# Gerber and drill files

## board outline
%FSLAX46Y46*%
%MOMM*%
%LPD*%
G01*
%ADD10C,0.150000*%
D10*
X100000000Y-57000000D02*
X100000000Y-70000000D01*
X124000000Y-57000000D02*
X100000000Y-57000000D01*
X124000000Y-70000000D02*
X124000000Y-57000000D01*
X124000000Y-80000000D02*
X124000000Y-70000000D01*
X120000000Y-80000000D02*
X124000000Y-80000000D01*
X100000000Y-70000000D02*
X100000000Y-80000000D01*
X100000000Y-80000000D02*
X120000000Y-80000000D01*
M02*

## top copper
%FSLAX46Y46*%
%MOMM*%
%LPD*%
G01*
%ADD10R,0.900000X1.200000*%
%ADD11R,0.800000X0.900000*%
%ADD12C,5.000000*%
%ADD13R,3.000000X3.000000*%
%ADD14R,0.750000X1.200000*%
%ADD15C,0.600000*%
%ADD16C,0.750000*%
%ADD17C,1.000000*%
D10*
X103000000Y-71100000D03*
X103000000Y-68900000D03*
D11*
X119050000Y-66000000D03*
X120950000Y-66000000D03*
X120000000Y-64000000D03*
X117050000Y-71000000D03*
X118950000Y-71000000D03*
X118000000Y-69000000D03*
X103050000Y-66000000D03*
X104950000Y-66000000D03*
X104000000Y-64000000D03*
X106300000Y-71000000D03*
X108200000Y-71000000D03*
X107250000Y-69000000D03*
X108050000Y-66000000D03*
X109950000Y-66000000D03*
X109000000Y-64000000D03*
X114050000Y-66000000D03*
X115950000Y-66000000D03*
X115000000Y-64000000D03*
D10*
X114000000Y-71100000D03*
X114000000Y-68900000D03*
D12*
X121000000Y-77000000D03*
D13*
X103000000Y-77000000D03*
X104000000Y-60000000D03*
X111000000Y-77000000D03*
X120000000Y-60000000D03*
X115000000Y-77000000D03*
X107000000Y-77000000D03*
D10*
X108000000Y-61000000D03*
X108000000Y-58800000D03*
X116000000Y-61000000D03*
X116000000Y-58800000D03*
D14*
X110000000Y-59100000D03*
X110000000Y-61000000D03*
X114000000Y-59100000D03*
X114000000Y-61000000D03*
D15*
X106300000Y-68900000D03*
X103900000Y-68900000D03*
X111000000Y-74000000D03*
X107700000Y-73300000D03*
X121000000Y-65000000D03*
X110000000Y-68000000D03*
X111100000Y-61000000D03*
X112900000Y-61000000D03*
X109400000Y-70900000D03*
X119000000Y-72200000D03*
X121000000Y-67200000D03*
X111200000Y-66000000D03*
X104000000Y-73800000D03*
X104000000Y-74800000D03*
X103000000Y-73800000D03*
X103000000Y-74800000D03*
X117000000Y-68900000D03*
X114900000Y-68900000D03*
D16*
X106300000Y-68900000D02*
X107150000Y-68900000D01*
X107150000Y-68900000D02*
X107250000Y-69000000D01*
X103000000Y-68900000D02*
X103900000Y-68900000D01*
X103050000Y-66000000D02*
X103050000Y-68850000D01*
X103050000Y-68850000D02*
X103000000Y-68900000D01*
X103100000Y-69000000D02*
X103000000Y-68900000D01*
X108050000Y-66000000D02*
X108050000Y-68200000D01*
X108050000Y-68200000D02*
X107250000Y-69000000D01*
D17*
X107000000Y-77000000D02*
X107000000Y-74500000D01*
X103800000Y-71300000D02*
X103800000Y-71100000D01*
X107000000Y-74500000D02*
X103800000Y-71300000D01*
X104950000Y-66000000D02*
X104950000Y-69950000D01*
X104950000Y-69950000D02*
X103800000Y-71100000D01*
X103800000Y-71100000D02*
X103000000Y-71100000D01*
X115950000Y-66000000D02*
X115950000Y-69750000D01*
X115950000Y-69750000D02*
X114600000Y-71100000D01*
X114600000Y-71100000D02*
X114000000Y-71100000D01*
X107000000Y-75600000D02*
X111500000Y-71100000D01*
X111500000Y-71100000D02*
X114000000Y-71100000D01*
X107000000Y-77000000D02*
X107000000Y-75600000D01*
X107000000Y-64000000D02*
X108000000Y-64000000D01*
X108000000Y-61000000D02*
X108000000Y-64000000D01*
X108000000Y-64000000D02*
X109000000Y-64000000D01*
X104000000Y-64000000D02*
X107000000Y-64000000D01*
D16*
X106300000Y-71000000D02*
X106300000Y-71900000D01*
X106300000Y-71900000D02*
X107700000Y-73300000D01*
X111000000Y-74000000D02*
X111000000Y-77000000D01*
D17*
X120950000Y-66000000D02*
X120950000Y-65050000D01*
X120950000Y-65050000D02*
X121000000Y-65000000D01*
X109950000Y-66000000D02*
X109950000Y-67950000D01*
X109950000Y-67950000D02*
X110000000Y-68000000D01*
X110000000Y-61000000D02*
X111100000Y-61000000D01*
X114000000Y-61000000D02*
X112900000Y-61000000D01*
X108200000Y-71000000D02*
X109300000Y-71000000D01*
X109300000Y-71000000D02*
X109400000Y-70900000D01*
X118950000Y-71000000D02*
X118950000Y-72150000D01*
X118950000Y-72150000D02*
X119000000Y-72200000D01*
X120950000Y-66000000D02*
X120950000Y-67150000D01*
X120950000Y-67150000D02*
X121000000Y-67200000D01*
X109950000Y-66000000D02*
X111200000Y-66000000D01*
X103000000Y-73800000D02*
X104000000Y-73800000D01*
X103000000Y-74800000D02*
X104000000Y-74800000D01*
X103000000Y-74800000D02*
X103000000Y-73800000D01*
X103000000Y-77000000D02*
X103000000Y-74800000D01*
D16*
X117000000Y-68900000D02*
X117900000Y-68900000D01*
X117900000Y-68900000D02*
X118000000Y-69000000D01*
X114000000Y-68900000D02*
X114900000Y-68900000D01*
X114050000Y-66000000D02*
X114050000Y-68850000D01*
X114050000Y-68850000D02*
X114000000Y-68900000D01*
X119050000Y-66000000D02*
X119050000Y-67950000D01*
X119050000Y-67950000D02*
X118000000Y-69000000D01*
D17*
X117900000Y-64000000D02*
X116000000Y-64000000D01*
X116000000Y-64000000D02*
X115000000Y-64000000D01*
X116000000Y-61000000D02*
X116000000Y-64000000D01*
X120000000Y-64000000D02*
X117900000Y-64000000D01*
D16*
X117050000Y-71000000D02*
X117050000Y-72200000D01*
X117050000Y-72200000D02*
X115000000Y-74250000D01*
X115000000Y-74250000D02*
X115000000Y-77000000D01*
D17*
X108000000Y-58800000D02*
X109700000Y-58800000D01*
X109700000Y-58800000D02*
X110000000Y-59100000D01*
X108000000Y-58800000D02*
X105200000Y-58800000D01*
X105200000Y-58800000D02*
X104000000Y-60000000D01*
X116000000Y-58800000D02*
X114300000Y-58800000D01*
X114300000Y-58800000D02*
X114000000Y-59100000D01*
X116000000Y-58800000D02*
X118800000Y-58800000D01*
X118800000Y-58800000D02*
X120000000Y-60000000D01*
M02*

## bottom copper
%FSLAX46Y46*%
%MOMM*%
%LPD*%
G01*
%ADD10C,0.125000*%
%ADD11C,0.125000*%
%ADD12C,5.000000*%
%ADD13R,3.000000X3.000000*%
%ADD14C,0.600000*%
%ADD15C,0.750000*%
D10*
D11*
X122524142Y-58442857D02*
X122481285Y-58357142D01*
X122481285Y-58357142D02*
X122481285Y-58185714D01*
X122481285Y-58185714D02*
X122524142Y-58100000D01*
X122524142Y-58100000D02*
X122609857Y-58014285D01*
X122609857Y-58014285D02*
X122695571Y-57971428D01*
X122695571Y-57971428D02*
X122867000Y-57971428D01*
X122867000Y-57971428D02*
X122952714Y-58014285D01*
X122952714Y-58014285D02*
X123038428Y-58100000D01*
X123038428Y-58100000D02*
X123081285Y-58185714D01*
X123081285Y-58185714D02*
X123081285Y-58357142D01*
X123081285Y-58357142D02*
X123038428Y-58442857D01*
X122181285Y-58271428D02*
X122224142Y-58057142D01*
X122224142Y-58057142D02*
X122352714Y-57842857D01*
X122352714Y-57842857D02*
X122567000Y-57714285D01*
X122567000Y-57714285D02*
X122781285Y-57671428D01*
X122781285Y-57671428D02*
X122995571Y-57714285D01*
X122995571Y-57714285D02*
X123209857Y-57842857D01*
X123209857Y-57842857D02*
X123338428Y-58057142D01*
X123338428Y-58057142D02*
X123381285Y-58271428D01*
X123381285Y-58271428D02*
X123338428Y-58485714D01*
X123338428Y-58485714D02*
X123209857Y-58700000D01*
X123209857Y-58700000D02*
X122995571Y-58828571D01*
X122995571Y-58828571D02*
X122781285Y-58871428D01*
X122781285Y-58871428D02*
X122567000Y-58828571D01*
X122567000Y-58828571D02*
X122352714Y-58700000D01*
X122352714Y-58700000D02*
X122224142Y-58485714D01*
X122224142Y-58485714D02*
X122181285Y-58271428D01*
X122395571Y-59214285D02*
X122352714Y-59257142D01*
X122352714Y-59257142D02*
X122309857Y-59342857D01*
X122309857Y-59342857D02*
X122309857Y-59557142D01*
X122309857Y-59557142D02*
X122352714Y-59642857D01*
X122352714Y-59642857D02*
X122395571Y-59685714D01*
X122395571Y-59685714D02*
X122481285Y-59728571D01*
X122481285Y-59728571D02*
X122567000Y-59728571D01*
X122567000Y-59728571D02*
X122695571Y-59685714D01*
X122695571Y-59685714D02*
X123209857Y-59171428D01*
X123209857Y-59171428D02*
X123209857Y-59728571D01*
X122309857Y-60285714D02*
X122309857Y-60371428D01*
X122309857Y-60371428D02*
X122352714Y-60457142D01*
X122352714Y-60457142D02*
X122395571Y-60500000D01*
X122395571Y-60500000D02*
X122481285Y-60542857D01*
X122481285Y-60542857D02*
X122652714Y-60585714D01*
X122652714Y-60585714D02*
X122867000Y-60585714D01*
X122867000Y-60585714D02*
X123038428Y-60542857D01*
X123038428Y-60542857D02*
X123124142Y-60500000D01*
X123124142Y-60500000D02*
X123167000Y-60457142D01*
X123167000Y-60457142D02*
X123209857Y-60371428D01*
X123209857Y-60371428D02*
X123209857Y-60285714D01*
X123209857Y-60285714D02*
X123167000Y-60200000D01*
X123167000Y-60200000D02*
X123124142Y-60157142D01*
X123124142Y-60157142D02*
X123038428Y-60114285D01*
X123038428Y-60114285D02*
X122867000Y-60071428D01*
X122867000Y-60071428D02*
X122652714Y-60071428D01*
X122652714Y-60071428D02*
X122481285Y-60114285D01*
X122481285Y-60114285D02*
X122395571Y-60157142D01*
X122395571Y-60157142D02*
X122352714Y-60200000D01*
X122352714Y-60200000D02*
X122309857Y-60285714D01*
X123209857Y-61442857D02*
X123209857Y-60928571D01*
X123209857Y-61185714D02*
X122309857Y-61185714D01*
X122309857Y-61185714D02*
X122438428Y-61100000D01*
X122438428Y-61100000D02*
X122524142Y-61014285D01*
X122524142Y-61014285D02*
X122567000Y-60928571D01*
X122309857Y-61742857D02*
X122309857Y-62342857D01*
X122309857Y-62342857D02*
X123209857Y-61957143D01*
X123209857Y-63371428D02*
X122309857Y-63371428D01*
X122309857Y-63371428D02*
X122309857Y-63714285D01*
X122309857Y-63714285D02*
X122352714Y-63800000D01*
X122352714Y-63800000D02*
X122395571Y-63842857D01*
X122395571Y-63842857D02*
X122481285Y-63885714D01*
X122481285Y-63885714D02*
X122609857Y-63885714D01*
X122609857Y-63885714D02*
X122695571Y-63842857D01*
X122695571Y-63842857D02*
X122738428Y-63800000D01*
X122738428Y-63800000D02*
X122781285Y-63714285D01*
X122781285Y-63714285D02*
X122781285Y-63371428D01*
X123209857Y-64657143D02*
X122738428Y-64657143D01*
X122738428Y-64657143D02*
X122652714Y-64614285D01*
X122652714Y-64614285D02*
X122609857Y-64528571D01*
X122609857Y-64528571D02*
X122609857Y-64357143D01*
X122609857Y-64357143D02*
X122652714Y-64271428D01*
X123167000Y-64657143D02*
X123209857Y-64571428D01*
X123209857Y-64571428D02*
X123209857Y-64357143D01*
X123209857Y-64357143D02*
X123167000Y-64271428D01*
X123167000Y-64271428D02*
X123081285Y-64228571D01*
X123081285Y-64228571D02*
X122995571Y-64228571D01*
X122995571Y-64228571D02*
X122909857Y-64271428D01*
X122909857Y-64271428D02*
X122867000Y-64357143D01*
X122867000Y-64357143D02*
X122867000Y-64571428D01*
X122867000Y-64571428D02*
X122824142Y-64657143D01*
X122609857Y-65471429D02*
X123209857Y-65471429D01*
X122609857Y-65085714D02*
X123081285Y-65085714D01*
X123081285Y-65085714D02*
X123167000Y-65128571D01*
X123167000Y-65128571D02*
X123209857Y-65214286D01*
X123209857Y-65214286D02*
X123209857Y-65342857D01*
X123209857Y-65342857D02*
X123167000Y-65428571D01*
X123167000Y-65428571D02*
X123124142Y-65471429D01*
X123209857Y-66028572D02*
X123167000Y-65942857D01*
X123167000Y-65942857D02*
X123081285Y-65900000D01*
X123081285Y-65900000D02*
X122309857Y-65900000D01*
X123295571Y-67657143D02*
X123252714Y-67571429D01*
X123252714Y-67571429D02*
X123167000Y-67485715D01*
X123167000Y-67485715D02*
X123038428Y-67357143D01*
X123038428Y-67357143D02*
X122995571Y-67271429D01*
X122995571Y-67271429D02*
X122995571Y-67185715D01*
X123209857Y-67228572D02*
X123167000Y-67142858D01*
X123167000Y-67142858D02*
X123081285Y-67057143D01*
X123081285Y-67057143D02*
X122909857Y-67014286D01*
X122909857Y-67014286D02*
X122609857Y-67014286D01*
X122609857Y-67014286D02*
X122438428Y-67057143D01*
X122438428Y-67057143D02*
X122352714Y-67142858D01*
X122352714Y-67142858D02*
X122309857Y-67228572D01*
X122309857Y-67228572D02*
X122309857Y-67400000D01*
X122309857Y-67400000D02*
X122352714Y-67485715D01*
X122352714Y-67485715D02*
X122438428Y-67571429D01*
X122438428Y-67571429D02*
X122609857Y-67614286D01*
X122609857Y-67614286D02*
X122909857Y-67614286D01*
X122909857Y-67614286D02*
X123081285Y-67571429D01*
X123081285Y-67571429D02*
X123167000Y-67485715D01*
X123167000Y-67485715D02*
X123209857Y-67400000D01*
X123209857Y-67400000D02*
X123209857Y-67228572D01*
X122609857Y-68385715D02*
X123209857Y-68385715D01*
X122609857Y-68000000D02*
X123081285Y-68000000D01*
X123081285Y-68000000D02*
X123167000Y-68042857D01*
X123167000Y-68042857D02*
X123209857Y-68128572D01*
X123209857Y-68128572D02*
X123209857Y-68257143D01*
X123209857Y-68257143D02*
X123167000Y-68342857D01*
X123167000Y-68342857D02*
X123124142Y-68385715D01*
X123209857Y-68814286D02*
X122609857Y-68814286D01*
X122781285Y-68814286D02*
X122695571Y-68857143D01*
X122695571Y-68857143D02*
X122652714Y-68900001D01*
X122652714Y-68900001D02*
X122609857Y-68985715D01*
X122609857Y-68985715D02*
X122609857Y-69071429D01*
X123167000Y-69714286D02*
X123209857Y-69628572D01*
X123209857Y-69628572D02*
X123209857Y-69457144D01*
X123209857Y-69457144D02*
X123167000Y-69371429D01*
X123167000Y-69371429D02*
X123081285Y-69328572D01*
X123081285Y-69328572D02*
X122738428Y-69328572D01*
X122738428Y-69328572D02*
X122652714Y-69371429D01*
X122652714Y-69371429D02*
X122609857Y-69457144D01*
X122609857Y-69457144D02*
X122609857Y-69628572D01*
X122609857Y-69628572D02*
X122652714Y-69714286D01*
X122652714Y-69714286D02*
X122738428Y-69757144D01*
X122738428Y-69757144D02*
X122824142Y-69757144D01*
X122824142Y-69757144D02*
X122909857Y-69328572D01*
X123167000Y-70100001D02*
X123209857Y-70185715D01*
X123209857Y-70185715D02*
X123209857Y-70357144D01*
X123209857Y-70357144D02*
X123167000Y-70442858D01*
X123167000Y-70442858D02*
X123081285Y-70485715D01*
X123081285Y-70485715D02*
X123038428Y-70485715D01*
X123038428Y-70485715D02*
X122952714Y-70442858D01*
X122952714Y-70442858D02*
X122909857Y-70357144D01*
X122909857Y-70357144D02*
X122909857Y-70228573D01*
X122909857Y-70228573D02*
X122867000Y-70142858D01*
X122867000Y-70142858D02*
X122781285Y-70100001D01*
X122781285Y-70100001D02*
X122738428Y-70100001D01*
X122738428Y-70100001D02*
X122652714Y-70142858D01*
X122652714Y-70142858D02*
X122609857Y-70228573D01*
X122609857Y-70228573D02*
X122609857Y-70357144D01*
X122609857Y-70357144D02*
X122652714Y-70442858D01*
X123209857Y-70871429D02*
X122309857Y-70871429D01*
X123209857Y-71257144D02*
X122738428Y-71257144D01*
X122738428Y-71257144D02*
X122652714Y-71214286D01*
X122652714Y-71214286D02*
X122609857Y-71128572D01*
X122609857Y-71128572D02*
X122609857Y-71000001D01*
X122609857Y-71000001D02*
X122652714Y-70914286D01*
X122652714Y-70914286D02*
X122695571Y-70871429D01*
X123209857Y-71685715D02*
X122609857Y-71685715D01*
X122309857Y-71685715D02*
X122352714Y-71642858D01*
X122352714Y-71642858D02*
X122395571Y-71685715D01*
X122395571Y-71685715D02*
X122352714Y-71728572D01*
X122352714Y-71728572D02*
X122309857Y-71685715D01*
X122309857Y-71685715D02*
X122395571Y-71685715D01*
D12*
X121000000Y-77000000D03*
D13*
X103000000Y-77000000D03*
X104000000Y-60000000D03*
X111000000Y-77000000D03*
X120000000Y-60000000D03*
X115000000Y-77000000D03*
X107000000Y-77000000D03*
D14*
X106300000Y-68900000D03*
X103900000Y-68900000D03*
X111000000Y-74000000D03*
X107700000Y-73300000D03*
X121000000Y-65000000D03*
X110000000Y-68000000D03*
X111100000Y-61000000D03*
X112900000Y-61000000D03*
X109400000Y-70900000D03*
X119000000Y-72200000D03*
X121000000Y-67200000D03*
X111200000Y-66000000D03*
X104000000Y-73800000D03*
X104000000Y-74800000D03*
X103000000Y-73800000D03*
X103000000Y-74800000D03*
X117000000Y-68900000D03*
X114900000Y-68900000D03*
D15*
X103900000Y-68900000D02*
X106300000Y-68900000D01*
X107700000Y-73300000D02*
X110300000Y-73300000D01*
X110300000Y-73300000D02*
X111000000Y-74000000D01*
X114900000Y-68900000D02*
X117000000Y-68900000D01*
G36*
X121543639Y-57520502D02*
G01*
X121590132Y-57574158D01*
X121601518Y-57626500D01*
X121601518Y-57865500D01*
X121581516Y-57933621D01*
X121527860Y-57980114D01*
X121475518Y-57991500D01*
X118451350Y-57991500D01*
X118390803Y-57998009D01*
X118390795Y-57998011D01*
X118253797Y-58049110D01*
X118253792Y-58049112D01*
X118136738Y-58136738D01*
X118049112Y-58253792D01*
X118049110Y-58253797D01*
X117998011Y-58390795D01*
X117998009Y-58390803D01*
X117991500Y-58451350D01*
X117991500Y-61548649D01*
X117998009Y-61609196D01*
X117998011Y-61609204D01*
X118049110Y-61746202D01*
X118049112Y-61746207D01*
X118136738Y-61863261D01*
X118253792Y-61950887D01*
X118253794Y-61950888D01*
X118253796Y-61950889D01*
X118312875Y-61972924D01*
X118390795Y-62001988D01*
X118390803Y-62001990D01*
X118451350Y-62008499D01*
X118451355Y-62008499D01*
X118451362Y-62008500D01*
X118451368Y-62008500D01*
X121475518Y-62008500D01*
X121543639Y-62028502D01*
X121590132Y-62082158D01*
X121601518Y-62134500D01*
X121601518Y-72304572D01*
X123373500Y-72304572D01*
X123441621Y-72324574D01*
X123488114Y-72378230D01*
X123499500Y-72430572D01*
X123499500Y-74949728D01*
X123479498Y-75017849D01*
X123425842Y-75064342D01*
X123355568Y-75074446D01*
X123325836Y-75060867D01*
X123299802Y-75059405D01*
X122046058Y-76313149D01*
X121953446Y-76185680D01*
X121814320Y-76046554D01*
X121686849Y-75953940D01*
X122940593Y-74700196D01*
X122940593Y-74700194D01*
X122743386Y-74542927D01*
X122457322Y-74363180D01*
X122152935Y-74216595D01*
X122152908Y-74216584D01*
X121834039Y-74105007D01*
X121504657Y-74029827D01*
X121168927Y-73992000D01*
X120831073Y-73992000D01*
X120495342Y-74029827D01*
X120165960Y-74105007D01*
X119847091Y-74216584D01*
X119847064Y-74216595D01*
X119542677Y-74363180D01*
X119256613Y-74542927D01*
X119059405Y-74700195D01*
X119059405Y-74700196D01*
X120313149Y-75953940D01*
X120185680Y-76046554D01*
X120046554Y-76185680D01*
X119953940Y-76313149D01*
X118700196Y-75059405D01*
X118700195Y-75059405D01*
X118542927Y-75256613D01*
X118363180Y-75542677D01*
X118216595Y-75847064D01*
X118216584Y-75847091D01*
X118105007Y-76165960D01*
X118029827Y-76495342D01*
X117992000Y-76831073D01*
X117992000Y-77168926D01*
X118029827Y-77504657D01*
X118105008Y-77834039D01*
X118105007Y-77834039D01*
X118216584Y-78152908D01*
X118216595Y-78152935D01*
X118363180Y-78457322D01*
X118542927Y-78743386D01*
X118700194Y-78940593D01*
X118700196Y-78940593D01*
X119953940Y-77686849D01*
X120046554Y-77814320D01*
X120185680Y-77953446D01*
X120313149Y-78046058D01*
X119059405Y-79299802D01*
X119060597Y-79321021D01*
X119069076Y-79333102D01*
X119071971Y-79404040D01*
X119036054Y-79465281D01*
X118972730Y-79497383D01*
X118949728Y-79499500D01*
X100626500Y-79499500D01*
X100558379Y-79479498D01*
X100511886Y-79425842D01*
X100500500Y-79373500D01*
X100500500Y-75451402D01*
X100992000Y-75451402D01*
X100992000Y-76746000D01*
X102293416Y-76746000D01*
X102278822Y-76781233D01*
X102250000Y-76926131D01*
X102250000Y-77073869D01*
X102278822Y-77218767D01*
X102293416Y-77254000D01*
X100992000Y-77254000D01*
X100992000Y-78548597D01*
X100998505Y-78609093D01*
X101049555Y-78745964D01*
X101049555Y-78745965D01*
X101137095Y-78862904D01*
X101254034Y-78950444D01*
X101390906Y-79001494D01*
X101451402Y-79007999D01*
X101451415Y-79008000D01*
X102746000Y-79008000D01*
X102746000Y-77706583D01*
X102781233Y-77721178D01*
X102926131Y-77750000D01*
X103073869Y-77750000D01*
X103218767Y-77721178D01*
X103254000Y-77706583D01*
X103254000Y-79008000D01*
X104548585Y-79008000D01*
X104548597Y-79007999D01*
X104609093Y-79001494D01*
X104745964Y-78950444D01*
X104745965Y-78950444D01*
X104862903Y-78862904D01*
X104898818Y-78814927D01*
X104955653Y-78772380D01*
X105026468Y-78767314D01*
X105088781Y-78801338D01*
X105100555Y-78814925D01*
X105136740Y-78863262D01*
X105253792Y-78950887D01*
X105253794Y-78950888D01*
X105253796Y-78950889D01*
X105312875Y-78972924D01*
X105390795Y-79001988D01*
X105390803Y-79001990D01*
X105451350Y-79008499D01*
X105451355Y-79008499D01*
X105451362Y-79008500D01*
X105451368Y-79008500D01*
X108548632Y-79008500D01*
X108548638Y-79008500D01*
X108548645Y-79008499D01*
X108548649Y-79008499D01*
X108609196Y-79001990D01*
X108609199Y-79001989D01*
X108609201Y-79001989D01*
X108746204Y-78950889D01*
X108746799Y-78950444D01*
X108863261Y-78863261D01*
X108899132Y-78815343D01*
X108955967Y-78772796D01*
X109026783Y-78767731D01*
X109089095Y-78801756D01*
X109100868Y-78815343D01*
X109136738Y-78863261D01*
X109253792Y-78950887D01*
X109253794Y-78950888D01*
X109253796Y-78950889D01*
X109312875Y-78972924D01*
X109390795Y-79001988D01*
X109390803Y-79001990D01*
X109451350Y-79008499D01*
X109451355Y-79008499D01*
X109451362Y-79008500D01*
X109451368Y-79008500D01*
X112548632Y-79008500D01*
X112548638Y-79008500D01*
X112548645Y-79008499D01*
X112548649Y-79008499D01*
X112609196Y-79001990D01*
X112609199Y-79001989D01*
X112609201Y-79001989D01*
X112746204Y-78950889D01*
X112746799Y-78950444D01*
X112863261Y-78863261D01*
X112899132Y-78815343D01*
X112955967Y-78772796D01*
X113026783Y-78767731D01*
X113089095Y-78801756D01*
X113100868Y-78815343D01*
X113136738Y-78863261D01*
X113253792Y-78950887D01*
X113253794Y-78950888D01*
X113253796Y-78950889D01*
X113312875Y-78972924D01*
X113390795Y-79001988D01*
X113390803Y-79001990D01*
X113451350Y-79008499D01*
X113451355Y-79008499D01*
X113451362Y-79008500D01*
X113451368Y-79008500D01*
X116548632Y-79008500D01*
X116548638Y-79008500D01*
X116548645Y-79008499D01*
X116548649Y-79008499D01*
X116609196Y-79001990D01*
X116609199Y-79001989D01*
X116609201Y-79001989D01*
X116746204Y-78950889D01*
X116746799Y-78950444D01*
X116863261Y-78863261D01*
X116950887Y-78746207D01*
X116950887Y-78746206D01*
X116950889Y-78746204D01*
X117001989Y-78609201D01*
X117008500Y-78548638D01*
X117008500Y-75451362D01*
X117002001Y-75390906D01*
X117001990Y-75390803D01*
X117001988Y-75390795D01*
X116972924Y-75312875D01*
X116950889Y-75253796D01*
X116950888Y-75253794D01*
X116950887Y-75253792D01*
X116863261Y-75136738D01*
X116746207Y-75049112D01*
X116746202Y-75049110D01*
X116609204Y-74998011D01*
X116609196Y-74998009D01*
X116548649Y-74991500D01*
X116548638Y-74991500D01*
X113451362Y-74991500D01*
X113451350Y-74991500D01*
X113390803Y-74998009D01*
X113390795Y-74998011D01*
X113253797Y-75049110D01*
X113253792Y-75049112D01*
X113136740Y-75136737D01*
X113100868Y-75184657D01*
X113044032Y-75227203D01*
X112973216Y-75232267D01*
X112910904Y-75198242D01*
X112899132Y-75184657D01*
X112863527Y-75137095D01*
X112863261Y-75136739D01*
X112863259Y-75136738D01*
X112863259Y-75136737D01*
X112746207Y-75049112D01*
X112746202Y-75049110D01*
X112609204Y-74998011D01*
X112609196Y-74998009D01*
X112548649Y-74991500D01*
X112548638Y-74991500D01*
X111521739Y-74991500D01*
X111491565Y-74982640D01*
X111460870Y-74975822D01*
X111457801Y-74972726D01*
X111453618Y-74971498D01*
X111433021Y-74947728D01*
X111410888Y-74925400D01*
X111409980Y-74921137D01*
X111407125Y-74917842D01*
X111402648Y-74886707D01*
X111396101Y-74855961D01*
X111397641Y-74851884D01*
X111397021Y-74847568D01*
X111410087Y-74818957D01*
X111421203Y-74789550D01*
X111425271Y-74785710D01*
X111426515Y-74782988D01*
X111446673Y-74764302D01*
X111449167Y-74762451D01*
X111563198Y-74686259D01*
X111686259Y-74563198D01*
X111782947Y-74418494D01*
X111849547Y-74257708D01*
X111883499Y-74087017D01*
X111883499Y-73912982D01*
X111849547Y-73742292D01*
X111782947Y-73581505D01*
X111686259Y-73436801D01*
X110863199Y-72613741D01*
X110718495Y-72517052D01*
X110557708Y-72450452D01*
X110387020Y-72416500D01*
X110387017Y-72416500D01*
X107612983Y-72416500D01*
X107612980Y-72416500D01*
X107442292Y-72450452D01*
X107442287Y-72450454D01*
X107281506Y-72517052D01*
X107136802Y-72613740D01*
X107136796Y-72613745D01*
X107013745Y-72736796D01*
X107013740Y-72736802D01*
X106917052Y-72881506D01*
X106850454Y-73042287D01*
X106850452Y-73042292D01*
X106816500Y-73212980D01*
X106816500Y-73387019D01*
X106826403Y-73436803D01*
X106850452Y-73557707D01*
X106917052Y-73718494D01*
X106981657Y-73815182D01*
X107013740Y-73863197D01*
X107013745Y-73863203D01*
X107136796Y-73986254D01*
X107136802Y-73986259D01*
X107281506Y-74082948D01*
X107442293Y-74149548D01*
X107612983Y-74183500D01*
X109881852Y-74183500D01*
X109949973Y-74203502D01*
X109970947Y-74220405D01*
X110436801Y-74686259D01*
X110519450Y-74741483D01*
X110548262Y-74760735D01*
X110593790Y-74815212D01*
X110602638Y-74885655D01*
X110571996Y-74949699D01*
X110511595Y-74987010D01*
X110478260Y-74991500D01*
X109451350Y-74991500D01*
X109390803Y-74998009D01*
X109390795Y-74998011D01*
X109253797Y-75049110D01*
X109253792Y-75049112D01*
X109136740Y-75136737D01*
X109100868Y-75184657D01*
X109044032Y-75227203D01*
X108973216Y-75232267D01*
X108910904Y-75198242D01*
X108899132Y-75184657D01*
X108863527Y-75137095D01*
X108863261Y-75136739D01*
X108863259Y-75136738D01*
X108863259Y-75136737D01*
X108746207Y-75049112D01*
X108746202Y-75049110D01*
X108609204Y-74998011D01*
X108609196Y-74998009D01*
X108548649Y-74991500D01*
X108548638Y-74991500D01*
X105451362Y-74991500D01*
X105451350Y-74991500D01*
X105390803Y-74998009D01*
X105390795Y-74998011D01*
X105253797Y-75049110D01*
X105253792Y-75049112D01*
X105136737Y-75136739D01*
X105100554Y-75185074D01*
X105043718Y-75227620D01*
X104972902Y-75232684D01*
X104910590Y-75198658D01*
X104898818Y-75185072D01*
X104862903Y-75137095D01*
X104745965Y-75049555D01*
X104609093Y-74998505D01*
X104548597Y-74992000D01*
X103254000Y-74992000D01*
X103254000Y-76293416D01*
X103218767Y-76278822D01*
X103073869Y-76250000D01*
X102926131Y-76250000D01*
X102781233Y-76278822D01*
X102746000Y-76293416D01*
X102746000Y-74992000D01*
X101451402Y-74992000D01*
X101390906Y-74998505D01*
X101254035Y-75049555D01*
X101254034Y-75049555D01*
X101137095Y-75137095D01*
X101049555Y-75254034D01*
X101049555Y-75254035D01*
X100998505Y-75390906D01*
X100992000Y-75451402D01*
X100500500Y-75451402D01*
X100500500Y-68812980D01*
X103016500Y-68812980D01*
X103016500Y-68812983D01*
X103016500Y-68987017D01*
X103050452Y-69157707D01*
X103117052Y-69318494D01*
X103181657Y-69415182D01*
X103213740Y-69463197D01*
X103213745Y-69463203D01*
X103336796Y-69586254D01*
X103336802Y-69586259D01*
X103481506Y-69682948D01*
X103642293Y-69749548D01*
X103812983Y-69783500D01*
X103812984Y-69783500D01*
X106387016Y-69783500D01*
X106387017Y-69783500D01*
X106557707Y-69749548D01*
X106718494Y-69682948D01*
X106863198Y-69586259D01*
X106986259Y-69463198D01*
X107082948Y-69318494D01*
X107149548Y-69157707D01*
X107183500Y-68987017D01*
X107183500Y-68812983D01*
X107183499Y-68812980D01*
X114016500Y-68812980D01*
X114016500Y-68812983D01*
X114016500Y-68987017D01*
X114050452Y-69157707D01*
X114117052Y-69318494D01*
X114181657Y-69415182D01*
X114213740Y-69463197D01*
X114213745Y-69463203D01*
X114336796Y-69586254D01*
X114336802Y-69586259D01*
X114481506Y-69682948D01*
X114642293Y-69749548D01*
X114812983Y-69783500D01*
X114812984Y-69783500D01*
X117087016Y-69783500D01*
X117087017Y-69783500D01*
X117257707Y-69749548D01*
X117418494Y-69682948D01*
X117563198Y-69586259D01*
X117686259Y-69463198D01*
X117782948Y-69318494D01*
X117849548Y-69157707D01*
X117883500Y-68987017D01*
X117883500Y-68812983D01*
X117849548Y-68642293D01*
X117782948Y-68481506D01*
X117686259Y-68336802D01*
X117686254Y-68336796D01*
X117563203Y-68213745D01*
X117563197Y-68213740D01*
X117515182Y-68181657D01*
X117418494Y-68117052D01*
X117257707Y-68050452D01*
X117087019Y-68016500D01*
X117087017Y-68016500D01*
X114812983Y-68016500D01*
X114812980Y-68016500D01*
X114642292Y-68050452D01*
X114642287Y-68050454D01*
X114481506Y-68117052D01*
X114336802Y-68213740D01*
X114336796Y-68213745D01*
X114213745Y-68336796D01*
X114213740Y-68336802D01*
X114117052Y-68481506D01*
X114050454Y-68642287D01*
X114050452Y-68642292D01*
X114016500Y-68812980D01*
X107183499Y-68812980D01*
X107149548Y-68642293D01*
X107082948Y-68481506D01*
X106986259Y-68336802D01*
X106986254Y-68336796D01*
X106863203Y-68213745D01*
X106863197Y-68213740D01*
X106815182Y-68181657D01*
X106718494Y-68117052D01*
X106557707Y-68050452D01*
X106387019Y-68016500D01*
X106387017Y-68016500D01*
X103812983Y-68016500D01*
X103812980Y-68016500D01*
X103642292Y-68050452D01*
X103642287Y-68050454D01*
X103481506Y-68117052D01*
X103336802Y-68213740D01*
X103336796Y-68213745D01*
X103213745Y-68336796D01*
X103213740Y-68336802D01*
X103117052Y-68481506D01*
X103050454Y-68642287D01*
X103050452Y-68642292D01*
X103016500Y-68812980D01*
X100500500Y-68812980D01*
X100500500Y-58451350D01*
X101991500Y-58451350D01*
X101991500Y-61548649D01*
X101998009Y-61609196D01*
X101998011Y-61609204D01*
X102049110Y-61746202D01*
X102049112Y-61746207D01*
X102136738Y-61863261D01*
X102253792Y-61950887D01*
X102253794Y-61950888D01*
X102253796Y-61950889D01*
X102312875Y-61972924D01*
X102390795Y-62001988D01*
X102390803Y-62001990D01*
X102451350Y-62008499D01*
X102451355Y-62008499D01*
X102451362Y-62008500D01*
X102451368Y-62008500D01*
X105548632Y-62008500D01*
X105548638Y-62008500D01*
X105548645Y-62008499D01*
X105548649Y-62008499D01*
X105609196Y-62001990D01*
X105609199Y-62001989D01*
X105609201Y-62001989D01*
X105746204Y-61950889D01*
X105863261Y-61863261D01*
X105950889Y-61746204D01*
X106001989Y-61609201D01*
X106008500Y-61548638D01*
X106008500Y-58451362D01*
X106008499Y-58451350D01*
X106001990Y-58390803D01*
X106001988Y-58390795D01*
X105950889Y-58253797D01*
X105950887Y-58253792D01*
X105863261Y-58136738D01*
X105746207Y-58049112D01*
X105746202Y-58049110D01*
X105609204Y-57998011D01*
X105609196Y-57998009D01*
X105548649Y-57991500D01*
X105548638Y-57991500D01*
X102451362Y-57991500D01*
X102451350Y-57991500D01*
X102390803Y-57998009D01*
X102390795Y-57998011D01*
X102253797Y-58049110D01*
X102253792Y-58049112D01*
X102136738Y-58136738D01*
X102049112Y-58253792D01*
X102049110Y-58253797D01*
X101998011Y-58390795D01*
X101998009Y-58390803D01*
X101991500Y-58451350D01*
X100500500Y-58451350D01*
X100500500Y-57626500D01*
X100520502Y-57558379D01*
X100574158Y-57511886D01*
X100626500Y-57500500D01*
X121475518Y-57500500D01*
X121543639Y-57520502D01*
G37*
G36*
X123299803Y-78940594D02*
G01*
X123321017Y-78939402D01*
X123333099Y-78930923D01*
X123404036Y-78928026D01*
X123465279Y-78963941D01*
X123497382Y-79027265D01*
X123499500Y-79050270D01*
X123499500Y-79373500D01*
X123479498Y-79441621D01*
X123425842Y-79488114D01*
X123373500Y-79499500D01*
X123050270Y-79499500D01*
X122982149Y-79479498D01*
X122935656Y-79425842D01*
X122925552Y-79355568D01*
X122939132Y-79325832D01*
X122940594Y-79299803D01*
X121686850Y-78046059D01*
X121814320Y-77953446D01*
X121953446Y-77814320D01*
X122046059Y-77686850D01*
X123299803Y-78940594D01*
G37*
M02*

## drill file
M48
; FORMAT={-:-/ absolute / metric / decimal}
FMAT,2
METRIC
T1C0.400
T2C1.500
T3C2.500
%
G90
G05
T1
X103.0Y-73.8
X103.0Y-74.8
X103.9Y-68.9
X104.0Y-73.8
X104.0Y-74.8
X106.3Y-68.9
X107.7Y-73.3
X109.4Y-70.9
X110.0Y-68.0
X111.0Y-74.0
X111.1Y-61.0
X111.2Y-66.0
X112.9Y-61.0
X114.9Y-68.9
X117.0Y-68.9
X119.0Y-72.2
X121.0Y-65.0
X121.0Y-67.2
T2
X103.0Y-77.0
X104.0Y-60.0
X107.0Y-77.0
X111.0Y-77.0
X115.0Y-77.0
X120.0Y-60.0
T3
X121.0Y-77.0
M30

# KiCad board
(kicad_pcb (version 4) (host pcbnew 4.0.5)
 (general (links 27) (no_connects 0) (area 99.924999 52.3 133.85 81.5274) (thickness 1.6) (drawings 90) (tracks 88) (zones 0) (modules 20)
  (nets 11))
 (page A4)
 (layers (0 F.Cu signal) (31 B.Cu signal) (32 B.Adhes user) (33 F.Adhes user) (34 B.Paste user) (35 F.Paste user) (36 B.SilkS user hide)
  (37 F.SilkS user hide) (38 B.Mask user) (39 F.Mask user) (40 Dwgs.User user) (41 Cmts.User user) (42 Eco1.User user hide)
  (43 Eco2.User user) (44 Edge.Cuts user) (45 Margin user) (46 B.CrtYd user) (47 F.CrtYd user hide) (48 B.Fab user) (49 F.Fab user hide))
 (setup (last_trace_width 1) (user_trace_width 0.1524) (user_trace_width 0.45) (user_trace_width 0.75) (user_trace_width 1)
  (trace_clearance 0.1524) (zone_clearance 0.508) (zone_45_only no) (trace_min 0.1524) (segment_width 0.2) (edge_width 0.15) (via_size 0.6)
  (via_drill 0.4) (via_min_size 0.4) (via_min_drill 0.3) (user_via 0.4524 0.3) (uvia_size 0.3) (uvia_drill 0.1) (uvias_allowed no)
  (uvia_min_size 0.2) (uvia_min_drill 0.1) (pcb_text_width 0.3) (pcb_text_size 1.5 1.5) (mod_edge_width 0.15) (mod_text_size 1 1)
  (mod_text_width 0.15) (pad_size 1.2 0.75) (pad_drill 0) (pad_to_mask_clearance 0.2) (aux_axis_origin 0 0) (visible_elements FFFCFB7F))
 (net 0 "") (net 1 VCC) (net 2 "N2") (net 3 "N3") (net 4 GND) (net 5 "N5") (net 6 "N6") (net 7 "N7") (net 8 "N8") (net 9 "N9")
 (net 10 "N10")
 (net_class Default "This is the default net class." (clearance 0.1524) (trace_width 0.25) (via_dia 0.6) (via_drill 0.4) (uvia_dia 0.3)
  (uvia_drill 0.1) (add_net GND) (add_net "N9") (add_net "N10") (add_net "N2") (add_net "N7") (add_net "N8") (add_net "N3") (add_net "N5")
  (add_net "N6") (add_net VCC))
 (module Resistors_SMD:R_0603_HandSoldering (layer F.Cu) (at 103 70 90)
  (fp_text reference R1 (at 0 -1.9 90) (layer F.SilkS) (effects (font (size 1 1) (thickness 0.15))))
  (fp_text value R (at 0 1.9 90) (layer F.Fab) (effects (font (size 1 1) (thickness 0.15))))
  (pad 1 smd rect (at -1.1 0 90) (size 1.2 0.9) (layers F.Cu F.Paste F.Mask) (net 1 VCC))
  (pad 2 smd rect (at 1.1 0 90) (size 1.2 0.9) (layers F.Cu F.Paste F.Mask) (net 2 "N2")))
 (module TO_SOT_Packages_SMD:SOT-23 (layer F.Cu) (at 120 65 90)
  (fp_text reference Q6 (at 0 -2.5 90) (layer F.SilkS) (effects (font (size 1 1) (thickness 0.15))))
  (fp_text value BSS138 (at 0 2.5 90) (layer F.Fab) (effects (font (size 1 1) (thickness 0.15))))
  (pad 1 smd rect (at -1 -0.95 90) (size 0.9 0.8) (layers F.Cu F.Paste F.Mask) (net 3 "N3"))
  (pad 2 smd rect (at -1 0.95 90) (size 0.9 0.8) (layers F.Cu F.Paste F.Mask) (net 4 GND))
  (pad 3 smd rect (at 1 0 90) (size 0.9 0.8) (layers F.Cu F.Paste F.Mask) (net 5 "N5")))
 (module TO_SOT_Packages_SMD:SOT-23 (layer F.Cu) (at 118 70 90)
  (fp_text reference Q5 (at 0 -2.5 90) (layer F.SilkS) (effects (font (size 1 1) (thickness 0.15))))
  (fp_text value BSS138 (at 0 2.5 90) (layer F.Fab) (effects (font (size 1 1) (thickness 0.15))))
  (pad 1 smd rect (at -1 -0.95 90) (size 0.9 0.8) (layers F.Cu F.Paste F.Mask) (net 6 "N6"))
  (pad 2 smd rect (at -1 0.95 90) (size 0.9 0.8) (layers F.Cu F.Paste F.Mask) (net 4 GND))
  (pad 3 smd rect (at 1 0 90) (size 0.9 0.8) (layers F.Cu F.Paste F.Mask) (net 3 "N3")))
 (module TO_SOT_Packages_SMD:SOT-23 (layer F.Cu) (at 104 65 90)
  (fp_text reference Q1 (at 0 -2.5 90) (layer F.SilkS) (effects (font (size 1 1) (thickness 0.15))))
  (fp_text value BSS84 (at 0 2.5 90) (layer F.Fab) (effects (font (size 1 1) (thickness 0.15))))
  (pad 1 smd rect (at -1 -0.95 90) (size 0.9 0.8) (layers F.Cu F.Paste F.Mask) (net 2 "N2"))
  (pad 2 smd rect (at -1 0.95 90) (size 0.9 0.8) (layers F.Cu F.Paste F.Mask) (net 1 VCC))
  (pad 3 smd rect (at 1 0 90) (size 0.9 0.8) (layers F.Cu F.Paste F.Mask) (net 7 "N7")))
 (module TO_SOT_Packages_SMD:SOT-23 (layer F.Cu) (at 107.25 70 90)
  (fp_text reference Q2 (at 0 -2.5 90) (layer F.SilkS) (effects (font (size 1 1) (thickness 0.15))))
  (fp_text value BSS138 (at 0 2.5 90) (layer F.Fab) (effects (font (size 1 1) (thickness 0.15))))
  (pad 1 smd rect (at -1 -0.95 90) (size 0.9 0.8) (layers F.Cu F.Paste F.Mask) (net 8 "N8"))
  (pad 2 smd rect (at -1 0.95 90) (size 0.9 0.8) (layers F.Cu F.Paste F.Mask) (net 4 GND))
  (pad 3 smd rect (at 1 0 90) (size 0.9 0.8) (layers F.Cu F.Paste F.Mask) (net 2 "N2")))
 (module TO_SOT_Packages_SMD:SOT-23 (layer F.Cu) (at 109 65 90)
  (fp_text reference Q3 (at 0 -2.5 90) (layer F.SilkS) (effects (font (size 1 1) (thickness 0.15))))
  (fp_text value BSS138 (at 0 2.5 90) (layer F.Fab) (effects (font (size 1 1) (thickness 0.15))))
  (pad 1 smd rect (at -1 -0.95 90) (size 0.9 0.8) (layers F.Cu F.Paste F.Mask) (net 2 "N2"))
  (pad 2 smd rect (at -1 0.95 90) (size 0.9 0.8) (layers F.Cu F.Paste F.Mask) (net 4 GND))
  (pad 3 smd rect (at 1 0 90) (size 0.9 0.8) (layers F.Cu F.Paste F.Mask) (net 7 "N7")))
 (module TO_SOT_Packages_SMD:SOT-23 (layer F.Cu) (at 115 65 90)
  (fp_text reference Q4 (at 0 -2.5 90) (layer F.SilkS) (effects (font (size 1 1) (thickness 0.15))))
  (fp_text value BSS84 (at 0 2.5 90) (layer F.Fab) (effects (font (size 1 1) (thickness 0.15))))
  (pad 1 smd rect (at -1 -0.95 90) (size 0.9 0.8) (layers F.Cu F.Paste F.Mask) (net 3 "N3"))
  (pad 2 smd rect (at -1 0.95 90) (size 0.9 0.8) (layers F.Cu F.Paste F.Mask) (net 1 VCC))
  (pad 3 smd rect (at 1 0 90) (size 0.9 0.8) (layers F.Cu F.Paste F.Mask) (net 5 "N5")))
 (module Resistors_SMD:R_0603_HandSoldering (layer F.Cu) (at 114 70 90)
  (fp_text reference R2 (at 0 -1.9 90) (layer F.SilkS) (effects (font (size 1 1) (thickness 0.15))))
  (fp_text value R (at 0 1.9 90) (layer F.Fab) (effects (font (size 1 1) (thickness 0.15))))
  (pad 1 smd rect (at -1.1 0 90) (size 1.2 0.9) (layers F.Cu F.Paste F.Mask) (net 1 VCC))
  (pad 2 smd rect (at 1.1 0 90) (size 1.2 0.9) (layers F.Cu F.Paste F.Mask) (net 3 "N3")))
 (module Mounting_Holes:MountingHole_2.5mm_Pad (layer F.Cu) (at 121 77)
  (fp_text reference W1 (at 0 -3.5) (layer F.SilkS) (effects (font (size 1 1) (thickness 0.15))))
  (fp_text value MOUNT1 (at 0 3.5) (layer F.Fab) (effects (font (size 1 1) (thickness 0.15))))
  (pad 1 thru_hole circle (at 0 0) (size 5 5) (drill 2.5) (layers *.Cu *.Mask) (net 4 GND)))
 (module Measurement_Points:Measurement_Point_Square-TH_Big (layer F.Cu) (at 103 77)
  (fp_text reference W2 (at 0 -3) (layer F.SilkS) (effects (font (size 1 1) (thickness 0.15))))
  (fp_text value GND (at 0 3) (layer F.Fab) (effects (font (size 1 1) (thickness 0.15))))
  (pad 1 thru_hole rect (at 0 0) (size 3 3) (drill 1.5) (layers *.Cu *.Mask) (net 4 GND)))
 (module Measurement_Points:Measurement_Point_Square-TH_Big (layer F.Cu) (at 104 60)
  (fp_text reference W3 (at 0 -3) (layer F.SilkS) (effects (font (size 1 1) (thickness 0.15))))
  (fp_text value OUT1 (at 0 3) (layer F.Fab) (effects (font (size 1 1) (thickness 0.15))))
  (pad 1 thru_hole rect (at 0 0) (size 3 3) (drill 1.5) (layers *.Cu *.Mask) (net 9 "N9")))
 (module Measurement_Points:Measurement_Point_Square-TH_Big (layer F.Cu) (at 111 77)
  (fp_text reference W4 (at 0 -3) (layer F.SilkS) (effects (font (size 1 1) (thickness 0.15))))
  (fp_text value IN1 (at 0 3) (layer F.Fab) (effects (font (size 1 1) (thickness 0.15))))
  (pad 1 thru_hole rect (at 0 0) (size 3 3) (drill 1.5) (layers *.Cu *.Mask) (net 8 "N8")))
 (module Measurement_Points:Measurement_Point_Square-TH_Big (layer F.Cu) (at 120 60)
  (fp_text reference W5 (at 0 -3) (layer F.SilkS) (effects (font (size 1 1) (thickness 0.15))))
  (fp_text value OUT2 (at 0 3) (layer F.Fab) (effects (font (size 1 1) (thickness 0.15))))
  (pad 1 thru_hole rect (at 0 0) (size 3 3) (drill 1.5) (layers *.Cu *.Mask) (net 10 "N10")))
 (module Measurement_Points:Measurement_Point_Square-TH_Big (layer F.Cu) (at 115 77)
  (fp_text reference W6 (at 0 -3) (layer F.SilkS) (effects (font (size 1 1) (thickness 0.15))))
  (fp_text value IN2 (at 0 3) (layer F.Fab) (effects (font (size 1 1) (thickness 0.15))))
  (pad 1 thru_hole rect (at 0 0) (size 3 3) (drill 1.5) (layers *.Cu *.Mask) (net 6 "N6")))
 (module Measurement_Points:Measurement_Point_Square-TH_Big (layer F.Cu) (at 107 77)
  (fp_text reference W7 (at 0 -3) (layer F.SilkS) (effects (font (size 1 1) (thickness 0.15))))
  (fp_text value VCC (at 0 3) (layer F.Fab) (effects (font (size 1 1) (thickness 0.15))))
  (pad 1 thru_hole rect (at 0 0) (size 3 3) (drill 1.5) (layers *.Cu *.Mask) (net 1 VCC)))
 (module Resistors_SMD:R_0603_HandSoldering (layer F.Cu) (at 108 59.9 90)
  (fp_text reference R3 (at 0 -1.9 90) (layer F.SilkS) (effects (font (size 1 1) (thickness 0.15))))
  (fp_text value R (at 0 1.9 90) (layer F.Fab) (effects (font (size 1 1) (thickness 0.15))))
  (pad 1 smd rect (at -1.1 0 90) (size 1.2 0.9) (layers F.Cu F.Paste F.Mask) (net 7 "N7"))
  (pad 2 smd rect (at 1.1 0 90) (size 1.2 0.9) (layers F.Cu F.Paste F.Mask) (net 9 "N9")))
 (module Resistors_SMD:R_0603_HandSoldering (layer F.Cu) (at 116 59.9 90)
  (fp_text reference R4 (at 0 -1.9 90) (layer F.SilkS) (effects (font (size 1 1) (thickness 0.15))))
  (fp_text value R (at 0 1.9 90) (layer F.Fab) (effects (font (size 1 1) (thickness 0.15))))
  (pad 1 smd rect (at -1.1 0 90) (size 1.2 0.9) (layers F.Cu F.Paste F.Mask) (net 5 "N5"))
  (pad 2 smd rect (at 1.1 0 90) (size 1.2 0.9) (layers F.Cu F.Paste F.Mask) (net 10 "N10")))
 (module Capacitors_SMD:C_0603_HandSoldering (layer F.Cu) (at 110 60.05 270)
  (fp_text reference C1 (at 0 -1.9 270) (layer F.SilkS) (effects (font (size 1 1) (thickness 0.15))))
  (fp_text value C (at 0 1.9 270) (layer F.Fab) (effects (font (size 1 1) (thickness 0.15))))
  (pad 1 smd rect (at -0.95 0 270) (size 1.2 0.75) (layers F.Cu F.Paste F.Mask) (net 9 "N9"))
  (pad 2 smd rect (at 0.95 0 270) (size 1.2 0.75) (layers F.Cu F.Paste F.Mask) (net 4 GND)))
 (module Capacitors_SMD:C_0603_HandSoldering (layer F.Cu) (at 114 60.05 270)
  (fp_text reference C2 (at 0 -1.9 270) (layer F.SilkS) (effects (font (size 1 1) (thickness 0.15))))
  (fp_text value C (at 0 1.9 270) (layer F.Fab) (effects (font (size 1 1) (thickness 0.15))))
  (pad 1 smd rect (at -0.95 0 270) (size 1.2 0.75) (layers F.Cu F.Paste F.Mask) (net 10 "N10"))
  (pad 2 smd rect (at 0.95 0 270) (size 1.2 0.75) (layers F.Cu F.Paste F.Mask) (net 4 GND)))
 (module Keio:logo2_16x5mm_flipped (layer F.Cu) (at 112 65.1)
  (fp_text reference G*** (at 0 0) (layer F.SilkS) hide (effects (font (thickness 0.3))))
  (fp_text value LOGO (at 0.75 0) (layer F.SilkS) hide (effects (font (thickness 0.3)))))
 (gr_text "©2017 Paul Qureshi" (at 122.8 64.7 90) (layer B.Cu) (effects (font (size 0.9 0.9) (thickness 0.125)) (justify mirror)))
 (gr_line (start 100 57) (end 100 70) (layer Edge.Cuts) (width 0.15))
 (gr_line (start 124 57) (end 100 57) (layer Edge.Cuts) (width 0.15))
 (gr_line (start 124 70) (end 124 57) (layer Edge.Cuts) (width 0.15))
 (gr_line (start 124 80) (end 124 70) (layer Edge.Cuts) (width 0.15))
 (gr_line (start 120 80) (end 124 80) (layer Edge.Cuts) (width 0.15))
 (gr_line (start 100 70) (end 100 80) (layer Edge.Cuts) (width 0.15))
 (gr_line (start 100 80) (end 120 80) (layer Edge.Cuts) (width 0.15))
 (segment (start 106.3 68.9) (end 107.15 68.9) (width 0.75) (layer F.Cu) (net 2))
 (segment (start 107.15 68.9) (end 107.25 69) (width 0.75) (layer F.Cu) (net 2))
 (segment (start 103.9 68.9) (end 106.3 68.9) (width 0.75) (layer B.Cu) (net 2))
 (via (at 106.3 68.9) (size 0.6) (drill 0.4) (layers F.Cu B.Cu) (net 2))
 (segment (start 103 68.9) (end 103.9 68.9) (width 0.75) (layer F.Cu) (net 2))
 (via (at 103.9 68.9) (size 0.6) (drill 0.4) (layers F.Cu B.Cu) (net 2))
 (segment (start 103.05 66) (end 103.05 68.85) (width 0.75) (layer F.Cu) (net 2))
 (segment (start 103.05 68.85) (end 103 68.9) (width 0.75) (layer F.Cu) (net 2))
 (segment (start 103.1 69) (end 103 68.9) (width 0.75) (layer F.Cu) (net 2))
 (segment (start 108.05 66) (end 108.05 68.2) (width 0.75) (layer F.Cu) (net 2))
 (segment (start 108.05 68.2) (end 107.25 69) (width 0.75) (layer F.Cu) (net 2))
 (segment (start 107 77) (end 107 74.5) (width 1) (layer F.Cu) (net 1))
 (segment (start 103.8 71.3) (end 103.8 71.1) (width 1) (layer F.Cu) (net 1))
 (segment (start 107 74.5) (end 103.8 71.3) (width 1) (layer F.Cu) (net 1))
 (segment (start 104.95 66) (end 104.95 69.95) (width 1) (layer F.Cu) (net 1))
 (segment (start 104.95 69.95) (end 103.8 71.1) (width 1) (layer F.Cu) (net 1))
 (segment (start 103.8 71.1) (end 103 71.1) (width 1) (layer F.Cu) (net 1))
 (segment (start 115.95 66) (end 115.95 69.75) (width 1) (layer F.Cu) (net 1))
 (segment (start 115.95 69.75) (end 114.6 71.1) (width 1) (layer F.Cu) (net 1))
 (segment (start 114.6 71.1) (end 114 71.1) (width 1) (layer F.Cu) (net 1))
 (segment (start 107 75.6) (end 111.5 71.1) (width 1) (layer F.Cu) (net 1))
 (segment (start 111.5 71.1) (end 114 71.1) (width 1) (layer F.Cu) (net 1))
 (segment (start 107 77) (end 107 75.6) (width 1) (layer F.Cu) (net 1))
 (segment (start 107 64) (end 108 64) (width 1) (layer F.Cu) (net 7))
 (segment (start 108 61) (end 108 64) (width 1) (layer F.Cu) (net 7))
 (segment (start 108 64) (end 109 64) (width 1) (layer F.Cu) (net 7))
 (segment (start 104 64) (end 107 64) (width 1) (layer F.Cu) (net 7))
 (segment (start 107.7 73.3) (end 110.3 73.3) (width 0.75) (layer B.Cu) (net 8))
 (segment (start 110.3 73.3) (end 111 74) (width 0.75) (layer B.Cu) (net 8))
 (via (at 111 74) (size 0.6) (drill 0.4) (layers F.Cu B.Cu) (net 8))
 (segment (start 106.3 71) (end 106.3 71.9) (width 0.75) (layer F.Cu) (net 8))
 (segment (start 106.3 71.9) (end 107.7 73.3) (width 0.75) (layer F.Cu) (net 8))
 (via (at 107.7 73.3) (size 0.6) (drill 0.4) (layers F.Cu B.Cu) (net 8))
 (segment (start 111 74) (end 111 77) (width 0.75) (layer F.Cu) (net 8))
 (segment (start 120.95 66) (end 120.95 65.05) (width 1) (layer F.Cu) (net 4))
 (segment (start 120.95 65.05) (end 121 65) (width 1) (layer F.Cu) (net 4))
 (via (at 121 65) (size 0.6) (drill 0.4) (layers F.Cu B.Cu) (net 4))
 (segment (start 109.95 66) (end 109.95 67.95) (width 1) (layer F.Cu) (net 4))
 (segment (start 109.95 67.95) (end 110 68) (width 1) (layer F.Cu) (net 4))
 (via (at 110 68) (size 0.6) (drill 0.4) (layers F.Cu B.Cu) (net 4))
 (segment (start 110 61) (end 111.1 61) (width 1) (layer F.Cu) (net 4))
 (via (at 111.1 61) (size 0.6) (drill 0.4) (layers F.Cu B.Cu) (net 4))
 (segment (start 114 61) (end 112.9 61) (width 1) (layer F.Cu) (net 4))
 (via (at 112.9 61) (size 0.6) (drill 0.4) (layers F.Cu B.Cu) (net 4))
 (segment (start 108.2 71) (end 109.3 71) (width 1) (layer F.Cu) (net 4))
 (segment (start 109.3 71) (end 109.4 70.9) (width 1) (layer F.Cu) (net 4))
 (via (at 109.4 70.9) (size 0.6) (drill 0.4) (layers F.Cu B.Cu) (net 4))
 (segment (start 118.95 71) (end 118.95 72.15) (width 1) (layer F.Cu) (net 4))
 (segment (start 118.95 72.15) (end 119 72.2) (width 1) (layer F.Cu) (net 4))
 (via (at 119 72.2) (size 0.6) (drill 0.4) (layers F.Cu B.Cu) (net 4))
 (segment (start 120.95 66) (end 120.95 67.15) (width 1) (layer F.Cu) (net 4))
 (segment (start 120.95 67.15) (end 121 67.2) (width 1) (layer F.Cu) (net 4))
 (via (at 121 67.2) (size 0.6) (drill 0.4) (layers F.Cu B.Cu) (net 4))
 (segment (start 109.95 66) (end 111.2 66) (width 1) (layer F.Cu) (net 4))
 (via (at 111.2 66) (size 0.6) (drill 0.4) (layers F.Cu B.Cu) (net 4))
 (segment (start 103 73.8) (end 104 73.8) (width 1) (layer F.Cu) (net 4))
 (via (at 104 73.8) (size 0.6) (drill 0.4) (layers F.Cu B.Cu) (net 4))
 (segment (start 103 74.8) (end 104 74.8) (width 1) (layer F.Cu) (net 4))
 (via (at 104 74.8) (size 0.6) (drill 0.4) (layers F.Cu B.Cu) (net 4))
 (segment (start 103 74.8) (end 103 73.8) (width 1) (layer F.Cu) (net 4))
 (via (at 103 73.8) (size 0.6) (drill 0.4) (layers F.Cu B.Cu) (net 4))
 (segment (start 103 77) (end 103 74.8) (width 1) (layer F.Cu) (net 4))
 (via (at 103 74.8) (size 0.6) (drill 0.4) (layers F.Cu B.Cu) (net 4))
 (segment (start 117 68.9) (end 117.9 68.9) (width 0.75) (layer F.Cu) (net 3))
 (segment (start 117.9 68.9) (end 118 69) (width 0.75) (layer F.Cu) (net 3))
 (segment (start 114.9 68.9) (end 117 68.9) (width 0.75) (layer B.Cu) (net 3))
 (via (at 117 68.9) (size 0.6) (drill 0.4) (layers F.Cu B.Cu) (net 3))
 (segment (start 114 68.9) (end 114.9 68.9) (width 0.75) (layer F.Cu) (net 3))
 (via (at 114.9 68.9) (size 0.6) (drill 0.4) (layers F.Cu B.Cu) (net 3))
 (segment (start 114.05 66) (end 114.05 68.85) (width 0.75) (layer F.Cu) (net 3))
 (segment (start 114.05 68.85) (end 114 68.9) (width 0.75) (layer F.Cu) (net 3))
 (segment (start 119.05 66) (end 119.05 67.95) (width 0.75) (layer F.Cu) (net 3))
 (segment (start 119.05 67.95) (end 118 69) (width 0.75) (layer F.Cu) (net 3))
 (segment (start 117.9 64) (end 116 64) (width 1) (layer F.Cu) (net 5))
 (segment (start 116 64) (end 115 64) (width 1) (layer F.Cu) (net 5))
 (segment (start 116 61) (end 116 64) (width 1) (layer F.Cu) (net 5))
 (segment (start 120 64) (end 117.9 64) (width 1) (layer F.Cu) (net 5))
 (segment (start 117.05 71) (end 117.05 72.2) (width 0.75) (layer F.Cu) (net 6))
 (segment (start 117.05 72.2) (end 115 74.25) (width 0.75) (layer F.Cu) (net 6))
 (segment (start 115 74.25) (end 115 77) (width 0.75) (layer F.Cu) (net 6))
 (segment (start 108 58.8) (end 109.7 58.8) (width 1) (layer F.Cu) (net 9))
 (segment (start 109.7 58.8) (end 110 59.1) (width 1) (layer F.Cu) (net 9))
 (segment (start 108 58.8) (end 105.2 58.8) (width 1) (layer F.Cu) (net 9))
 (segment (start 105.2 58.8) (end 104 60) (width 1) (layer F.Cu) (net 9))
 (segment (start 116 58.8) (end 114.3 58.8) (width 1) (layer F.Cu) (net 10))
 (segment (start 114.3 58.8) (end 114 59.1) (width 1) (layer F.Cu) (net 10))
 (segment (start 116 58.8) (end 118.8 58.8) (width 1) (layer F.Cu) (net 10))
 (segment (start 118.8 58.8) (end 120 60) (width 1) (layer F.Cu) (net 10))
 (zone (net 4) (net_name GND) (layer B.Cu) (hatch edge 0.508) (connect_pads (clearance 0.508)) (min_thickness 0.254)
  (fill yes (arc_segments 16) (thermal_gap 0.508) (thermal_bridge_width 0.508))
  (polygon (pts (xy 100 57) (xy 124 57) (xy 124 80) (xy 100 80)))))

